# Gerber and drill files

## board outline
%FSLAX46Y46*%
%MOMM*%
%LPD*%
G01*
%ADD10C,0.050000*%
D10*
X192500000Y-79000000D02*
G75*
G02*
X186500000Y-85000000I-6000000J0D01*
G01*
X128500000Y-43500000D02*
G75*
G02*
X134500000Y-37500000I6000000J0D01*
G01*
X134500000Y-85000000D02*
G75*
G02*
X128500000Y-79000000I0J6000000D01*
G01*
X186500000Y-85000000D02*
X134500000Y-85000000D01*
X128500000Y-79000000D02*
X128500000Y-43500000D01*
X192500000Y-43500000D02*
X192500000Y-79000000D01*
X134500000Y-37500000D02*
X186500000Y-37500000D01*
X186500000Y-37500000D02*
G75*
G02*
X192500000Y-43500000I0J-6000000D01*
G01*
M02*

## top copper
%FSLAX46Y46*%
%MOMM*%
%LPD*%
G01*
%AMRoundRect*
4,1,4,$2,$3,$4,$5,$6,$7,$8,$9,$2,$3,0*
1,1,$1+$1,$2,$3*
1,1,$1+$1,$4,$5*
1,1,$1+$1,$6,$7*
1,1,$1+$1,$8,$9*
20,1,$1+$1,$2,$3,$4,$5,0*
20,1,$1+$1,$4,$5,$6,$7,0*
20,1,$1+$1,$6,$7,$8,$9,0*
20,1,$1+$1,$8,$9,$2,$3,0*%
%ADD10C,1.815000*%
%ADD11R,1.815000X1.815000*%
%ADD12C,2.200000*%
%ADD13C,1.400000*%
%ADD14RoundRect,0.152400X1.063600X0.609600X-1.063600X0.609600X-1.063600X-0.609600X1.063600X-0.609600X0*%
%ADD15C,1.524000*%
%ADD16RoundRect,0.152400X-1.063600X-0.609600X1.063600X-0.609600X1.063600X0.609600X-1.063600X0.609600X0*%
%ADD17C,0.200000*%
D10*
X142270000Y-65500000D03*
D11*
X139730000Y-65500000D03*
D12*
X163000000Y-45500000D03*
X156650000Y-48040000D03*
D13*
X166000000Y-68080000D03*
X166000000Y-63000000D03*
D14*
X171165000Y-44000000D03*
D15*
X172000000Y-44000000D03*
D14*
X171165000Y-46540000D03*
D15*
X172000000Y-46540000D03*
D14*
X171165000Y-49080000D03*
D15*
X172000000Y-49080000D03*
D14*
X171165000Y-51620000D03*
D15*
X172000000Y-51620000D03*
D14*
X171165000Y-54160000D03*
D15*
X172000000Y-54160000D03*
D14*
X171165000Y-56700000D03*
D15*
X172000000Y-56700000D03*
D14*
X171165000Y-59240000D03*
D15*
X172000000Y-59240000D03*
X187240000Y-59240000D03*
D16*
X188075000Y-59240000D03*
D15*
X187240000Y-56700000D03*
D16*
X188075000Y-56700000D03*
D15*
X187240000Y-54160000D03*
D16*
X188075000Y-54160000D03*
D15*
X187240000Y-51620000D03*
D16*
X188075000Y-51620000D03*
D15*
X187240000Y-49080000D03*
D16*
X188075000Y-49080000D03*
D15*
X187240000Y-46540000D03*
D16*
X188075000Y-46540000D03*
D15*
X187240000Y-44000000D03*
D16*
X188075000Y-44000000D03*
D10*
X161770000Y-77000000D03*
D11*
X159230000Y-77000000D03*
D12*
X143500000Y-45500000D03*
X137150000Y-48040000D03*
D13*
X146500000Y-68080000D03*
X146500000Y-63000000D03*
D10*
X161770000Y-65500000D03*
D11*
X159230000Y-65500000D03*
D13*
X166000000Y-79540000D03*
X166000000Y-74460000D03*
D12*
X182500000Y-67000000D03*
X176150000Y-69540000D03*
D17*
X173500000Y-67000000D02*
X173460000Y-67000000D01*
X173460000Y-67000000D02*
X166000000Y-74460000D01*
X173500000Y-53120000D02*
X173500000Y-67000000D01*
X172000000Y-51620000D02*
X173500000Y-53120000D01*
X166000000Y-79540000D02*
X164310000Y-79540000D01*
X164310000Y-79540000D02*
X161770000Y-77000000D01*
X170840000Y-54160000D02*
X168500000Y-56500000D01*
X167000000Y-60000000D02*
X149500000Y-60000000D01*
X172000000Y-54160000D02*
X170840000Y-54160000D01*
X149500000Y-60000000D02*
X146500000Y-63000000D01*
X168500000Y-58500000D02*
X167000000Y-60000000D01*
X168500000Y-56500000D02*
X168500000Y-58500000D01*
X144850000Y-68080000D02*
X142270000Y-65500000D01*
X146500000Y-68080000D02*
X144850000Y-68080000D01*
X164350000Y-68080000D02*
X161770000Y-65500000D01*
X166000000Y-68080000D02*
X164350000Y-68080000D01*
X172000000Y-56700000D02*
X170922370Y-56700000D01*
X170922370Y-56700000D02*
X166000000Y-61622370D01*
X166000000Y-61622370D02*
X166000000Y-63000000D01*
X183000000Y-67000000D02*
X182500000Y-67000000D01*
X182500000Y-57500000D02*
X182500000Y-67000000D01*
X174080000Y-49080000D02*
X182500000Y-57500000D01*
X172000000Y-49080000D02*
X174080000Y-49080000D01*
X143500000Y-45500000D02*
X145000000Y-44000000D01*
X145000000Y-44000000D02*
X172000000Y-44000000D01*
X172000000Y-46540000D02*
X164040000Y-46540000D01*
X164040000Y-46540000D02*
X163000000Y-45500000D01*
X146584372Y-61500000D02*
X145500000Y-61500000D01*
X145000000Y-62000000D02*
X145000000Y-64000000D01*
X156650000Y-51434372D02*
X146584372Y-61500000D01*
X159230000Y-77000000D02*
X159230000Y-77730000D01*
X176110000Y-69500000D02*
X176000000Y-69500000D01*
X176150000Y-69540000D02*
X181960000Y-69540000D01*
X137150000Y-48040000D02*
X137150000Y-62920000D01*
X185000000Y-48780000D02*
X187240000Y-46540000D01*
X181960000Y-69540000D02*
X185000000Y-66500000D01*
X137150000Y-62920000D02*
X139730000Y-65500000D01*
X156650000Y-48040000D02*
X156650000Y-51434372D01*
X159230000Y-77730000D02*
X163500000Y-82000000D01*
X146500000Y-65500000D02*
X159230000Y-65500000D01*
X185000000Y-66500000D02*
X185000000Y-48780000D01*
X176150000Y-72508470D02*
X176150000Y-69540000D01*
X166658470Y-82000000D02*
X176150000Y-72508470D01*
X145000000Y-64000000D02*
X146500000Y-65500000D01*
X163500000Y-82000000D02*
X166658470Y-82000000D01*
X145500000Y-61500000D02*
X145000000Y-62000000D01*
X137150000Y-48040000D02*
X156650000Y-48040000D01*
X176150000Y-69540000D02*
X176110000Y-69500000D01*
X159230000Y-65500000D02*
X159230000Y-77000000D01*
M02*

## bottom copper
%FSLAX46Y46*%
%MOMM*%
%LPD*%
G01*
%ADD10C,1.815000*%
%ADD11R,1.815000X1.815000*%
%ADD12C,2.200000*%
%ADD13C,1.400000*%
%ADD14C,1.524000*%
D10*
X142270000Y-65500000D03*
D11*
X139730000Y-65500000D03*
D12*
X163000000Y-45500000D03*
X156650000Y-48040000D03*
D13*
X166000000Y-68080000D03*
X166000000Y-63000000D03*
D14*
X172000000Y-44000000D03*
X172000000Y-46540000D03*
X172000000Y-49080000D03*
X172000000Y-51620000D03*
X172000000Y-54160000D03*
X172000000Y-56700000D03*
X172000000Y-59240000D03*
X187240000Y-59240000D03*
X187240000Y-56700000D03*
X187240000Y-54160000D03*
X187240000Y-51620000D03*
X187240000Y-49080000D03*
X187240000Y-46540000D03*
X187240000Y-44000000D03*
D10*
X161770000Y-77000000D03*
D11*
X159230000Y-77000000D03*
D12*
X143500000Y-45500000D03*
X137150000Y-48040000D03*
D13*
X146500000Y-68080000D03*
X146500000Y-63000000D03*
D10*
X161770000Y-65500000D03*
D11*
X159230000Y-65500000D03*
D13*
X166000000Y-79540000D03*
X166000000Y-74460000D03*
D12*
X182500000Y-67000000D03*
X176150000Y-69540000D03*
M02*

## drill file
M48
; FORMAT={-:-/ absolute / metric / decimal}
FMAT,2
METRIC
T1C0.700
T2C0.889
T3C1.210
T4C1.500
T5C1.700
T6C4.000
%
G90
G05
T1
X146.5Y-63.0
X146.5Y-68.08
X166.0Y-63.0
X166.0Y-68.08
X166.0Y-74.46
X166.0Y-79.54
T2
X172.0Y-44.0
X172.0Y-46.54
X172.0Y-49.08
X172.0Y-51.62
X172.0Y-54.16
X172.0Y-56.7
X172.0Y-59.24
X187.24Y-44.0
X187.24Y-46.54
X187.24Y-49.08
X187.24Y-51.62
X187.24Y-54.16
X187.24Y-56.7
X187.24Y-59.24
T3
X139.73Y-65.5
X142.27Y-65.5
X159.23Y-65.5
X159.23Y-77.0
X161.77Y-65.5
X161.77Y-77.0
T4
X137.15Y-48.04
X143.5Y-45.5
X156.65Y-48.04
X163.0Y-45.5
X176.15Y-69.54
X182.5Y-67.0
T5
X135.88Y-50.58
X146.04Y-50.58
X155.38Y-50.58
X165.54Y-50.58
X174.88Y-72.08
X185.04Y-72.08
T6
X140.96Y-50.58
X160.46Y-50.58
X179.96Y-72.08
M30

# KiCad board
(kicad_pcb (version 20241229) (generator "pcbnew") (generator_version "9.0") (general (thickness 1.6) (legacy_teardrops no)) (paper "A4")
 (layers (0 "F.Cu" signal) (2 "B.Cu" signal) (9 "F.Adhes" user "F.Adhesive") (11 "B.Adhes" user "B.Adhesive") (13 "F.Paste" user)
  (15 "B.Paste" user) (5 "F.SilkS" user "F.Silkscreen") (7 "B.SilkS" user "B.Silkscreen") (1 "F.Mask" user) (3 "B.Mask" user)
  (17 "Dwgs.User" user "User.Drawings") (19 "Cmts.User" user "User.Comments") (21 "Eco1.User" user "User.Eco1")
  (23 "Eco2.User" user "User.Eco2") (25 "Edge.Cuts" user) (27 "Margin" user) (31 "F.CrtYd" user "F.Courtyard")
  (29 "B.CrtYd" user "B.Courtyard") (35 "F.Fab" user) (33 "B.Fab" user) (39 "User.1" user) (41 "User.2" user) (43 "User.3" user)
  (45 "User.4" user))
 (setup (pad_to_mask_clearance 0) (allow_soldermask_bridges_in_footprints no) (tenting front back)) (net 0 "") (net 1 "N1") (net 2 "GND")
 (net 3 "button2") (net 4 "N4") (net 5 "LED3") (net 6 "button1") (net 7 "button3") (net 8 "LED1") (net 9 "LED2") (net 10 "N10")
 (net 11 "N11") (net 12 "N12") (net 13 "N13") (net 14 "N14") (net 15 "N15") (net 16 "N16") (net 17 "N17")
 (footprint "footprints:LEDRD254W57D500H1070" (layer "F.Cu") (at 141 65.5)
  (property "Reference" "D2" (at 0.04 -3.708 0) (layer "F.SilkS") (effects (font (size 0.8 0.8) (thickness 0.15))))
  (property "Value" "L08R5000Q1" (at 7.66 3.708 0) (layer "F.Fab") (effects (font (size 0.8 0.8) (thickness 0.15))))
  (pad "A" thru_hole circle (at 1.27 0) (size 1.815 1.815) (drill 1.21) (layers "*.Cu" "*.Mask") (remove_unused_layers no) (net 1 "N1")
   (solder_mask_margin 0.102))
  (pad "C" thru_hole rect (at -1.27 0) (size 1.815 1.815) (drill 1.21) (layers "*.Cu" "*.Mask") (remove_unused_layers no) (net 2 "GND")
   (solder_mask_margin 0.102)))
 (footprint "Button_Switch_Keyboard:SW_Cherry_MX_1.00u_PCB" (layer "F.Cu") (at 163 45.5)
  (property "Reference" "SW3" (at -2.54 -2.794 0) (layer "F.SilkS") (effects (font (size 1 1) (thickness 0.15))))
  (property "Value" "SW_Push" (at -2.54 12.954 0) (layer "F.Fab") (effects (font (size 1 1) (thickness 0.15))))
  (pad "" np_thru_hole circle (at -7.62 5.08) (size 1.7 1.7) (drill 1.7) (layers "*.Cu" "*.Mask"))
  (pad "" np_thru_hole circle (at -2.54 5.08) (size 4 4) (drill 4) (layers "*.Cu" "*.Mask"))
  (pad "" np_thru_hole circle (at 2.54 5.08) (size 1.7 1.7) (drill 1.7) (layers "*.Cu" "*.Mask"))
  (pad "1" thru_hole circle (at 0 0) (size 2.2 2.2) (drill 1.5) (layers "*.Cu" "*.Mask") (remove_unused_layers no) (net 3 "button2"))
  (pad "2" thru_hole circle (at -6.35 2.54) (size 2.2 2.2) (drill 1.5) (layers "*.Cu" "*.Mask") (remove_unused_layers no) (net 2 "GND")))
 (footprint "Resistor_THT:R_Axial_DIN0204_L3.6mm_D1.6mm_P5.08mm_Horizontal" (layer "F.Cu") (at 166 68.08 90)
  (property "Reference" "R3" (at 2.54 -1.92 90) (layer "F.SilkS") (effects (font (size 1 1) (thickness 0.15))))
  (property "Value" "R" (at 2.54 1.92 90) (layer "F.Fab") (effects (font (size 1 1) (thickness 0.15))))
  (pad "1" thru_hole circle (at 0 0 90) (size 1.4 1.4) (drill 0.7) (layers "*.Cu" "*.Mask") (remove_unused_layers no) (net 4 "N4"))
  (pad "2" thru_hole circle (at 5.08 0 90) (size 1.4 1.4) (drill 0.7) (layers "*.Cu" "*.Mask") (remove_unused_layers no) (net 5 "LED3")))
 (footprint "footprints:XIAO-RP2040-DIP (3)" (layer "F.Cu") (at 179.62 51.62)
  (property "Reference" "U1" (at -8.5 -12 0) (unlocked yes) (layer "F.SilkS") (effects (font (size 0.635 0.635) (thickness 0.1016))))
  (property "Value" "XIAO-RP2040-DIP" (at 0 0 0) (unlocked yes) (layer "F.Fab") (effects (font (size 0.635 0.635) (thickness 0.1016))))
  (pad "1" smd roundrect (at -8.455 -7.62 180) (size 2.432 1.524) (layers "F.Cu" "F.Mask") (roundrect_rratio 0.1) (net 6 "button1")
   (thermal_bridge_angle 45))
  (pad "1" thru_hole circle (at -7.62 -7.62 180) (size 1.524 1.524) (drill 0.889) (layers "*.Cu" "*.Mask") (remove_unused_layers no)
   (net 6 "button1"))
  (pad "2" smd roundrect (at -8.455 -5.08 180) (size 2.432 1.524) (layers "F.Cu" "F.Mask") (roundrect_rratio 0.1) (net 3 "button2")
   (thermal_bridge_angle 45))
  (pad "2" thru_hole circle (at -7.62 -5.08 180) (size 1.524 1.524) (drill 0.889) (layers "*.Cu" "*.Mask") (remove_unused_layers no)
   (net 3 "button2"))
  (pad "3" smd roundrect (at -8.455 -2.54 180) (size 2.432 1.524) (layers "F.Cu" "F.Mask") (roundrect_rratio 0.1) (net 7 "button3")
   (thermal_bridge_angle 45))
  (pad "3" thru_hole circle (at -7.62 -2.54 180) (size 1.524 1.524) (drill 0.889) (layers "*.Cu" "*.Mask") (remove_unused_layers no)
   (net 7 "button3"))
  (pad "4" smd roundrect (at -8.455 0 180) (size 2.432 1.524) (layers "F.Cu" "F.Mask") (roundrect_rratio 0.1) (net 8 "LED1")
   (thermal_bridge_angle 45))
  (pad "4" thru_hole circle (at -7.62 0 180) (size 1.524 1.524) (drill 0.889) (layers "*.Cu" "*.Mask") (remove_unused_layers no)
   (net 8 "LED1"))
  (pad "5" smd roundrect (at -8.455 2.54 180) (size 2.432 1.524) (layers "F.Cu" "F.Mask") (roundrect_rratio 0.1) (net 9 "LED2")
   (thermal_bridge_angle 45))
  (pad "5" thru_hole circle (at -7.62 2.54 180) (size 1.524 1.524) (drill 0.889) (layers "*.Cu" "*.Mask") (remove_unused_layers no)
   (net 9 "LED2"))
  (pad "6" smd roundrect (at -8.455 5.08 180) (size 2.432 1.524) (layers "F.Cu" "F.Mask") (roundrect_rratio 0.1) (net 5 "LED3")
   (thermal_bridge_angle 45))
  (pad "6" thru_hole circle (at -7.62 5.08 180) (size 1.524 1.524) (drill 0.889) (layers "*.Cu" "*.Mask") (remove_unused_layers no)
   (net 5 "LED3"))
  (pad "7" smd roundrect (at -8.455 7.62 180) (size 2.432 1.524) (layers "F.Cu" "F.Mask") (roundrect_rratio 0.1) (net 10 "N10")
   (thermal_bridge_angle 45))
  (pad "7" thru_hole circle (at -7.62 7.62 180) (size 1.524 1.524) (drill 0.889) (layers "*.Cu" "*.Mask") (remove_unused_layers no)
   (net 10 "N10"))
  (pad "8" thru_hole circle (at 7.62 7.62) (size 1.524 1.524) (drill 0.889) (layers "*.Cu" "*.Mask") (remove_unused_layers no)
   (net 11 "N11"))
  (pad "8" smd roundrect (at 8.455 7.62) (size 2.432 1.524) (layers "F.Cu" "F.Mask") (roundrect_rratio 0.1) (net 11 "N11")
   (thermal_bridge_angle 45))
  (pad "9" thru_hole circle (at 7.62 5.08) (size 1.524 1.524) (drill 0.889) (layers "*.Cu" "*.Mask") (remove_unused_layers no)
   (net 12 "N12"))
  (pad "9" smd roundrect (at 8.455 5.08) (size 2.432 1.524) (layers "F.Cu" "F.Mask") (roundrect_rratio 0.1) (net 12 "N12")
   (thermal_bridge_angle 45))
  (pad "10" thru_hole circle (at 7.62 2.54) (size 1.524 1.524) (drill 0.889) (layers "*.Cu" "*.Mask") (remove_unused_layers no)
   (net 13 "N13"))
  (pad "10" smd roundrect (at 8.455 2.54) (size 2.432 1.524) (layers "F.Cu" "F.Mask") (roundrect_rratio 0.1) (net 13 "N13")
   (thermal_bridge_angle 45))
  (pad "11" thru_hole circle (at 7.62 0) (size 1.524 1.524) (drill 0.889) (layers "*.Cu" "*.Mask") (remove_unused_layers no) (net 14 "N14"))
  (pad "11" smd roundrect (at 8.455 0) (size 2.432 1.524) (layers "F.Cu" "F.Mask") (roundrect_rratio 0.1) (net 14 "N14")
   (thermal_bridge_angle 45))
  (pad "12" thru_hole circle (at 7.62 -2.54) (size 1.524 1.524) (drill 0.889) (layers "*.Cu" "*.Mask") (remove_unused_layers no)
   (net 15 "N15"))
  (pad "12" smd roundrect (at 8.455 -2.54) (size 2.432 1.524) (layers "F.Cu" "F.Mask") (roundrect_rratio 0.1) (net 15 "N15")
   (thermal_bridge_angle 45))
  (pad "13" thru_hole circle (at 7.62 -5.08) (size 1.524 1.524) (drill 0.889) (layers "*.Cu" "*.Mask") (remove_unused_layers no)
   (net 2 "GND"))
  (pad "13" smd roundrect (at 8.455 -5.08) (size 2.432 1.524) (layers "F.Cu" "F.Mask") (roundrect_rratio 0.1) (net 2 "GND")
   (thermal_bridge_angle 45))
  (pad "14" thru_hole circle (at 7.62 -7.62) (size 1.524 1.524) (drill 0.889) (layers "*.Cu" "*.Mask") (remove_unused_layers no)
   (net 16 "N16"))
  (pad "14" smd roundrect (at 8.455 -7.62) (size 2.432 1.524) (layers "F.Cu" "F.Mask") (roundrect_rratio 0.1) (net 16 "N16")
   (thermal_bridge_angle 45)))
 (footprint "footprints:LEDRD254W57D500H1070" (layer "F.Cu") (at 160.5 77)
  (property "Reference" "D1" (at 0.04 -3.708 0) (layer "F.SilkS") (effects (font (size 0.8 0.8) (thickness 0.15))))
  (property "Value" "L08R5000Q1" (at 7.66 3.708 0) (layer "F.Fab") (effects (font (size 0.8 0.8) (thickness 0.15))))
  (pad "A" thru_hole circle (at 1.27 0) (size 1.815 1.815) (drill 1.21) (layers "*.Cu" "*.Mask") (remove_unused_layers no) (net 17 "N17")
   (solder_mask_margin 0.102))
  (pad "C" thru_hole rect (at -1.27 0) (size 1.815 1.815) (drill 1.21) (layers "*.Cu" "*.Mask") (remove_unused_layers no) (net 2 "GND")
   (solder_mask_margin 0.102)))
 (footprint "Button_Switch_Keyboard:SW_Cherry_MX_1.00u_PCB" (layer "F.Cu") (at 143.5 45.5)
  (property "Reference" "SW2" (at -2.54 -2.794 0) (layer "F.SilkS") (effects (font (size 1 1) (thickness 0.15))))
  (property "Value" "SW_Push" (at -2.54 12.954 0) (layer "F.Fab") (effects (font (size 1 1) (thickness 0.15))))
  (pad "" np_thru_hole circle (at -7.62 5.08) (size 1.7 1.7) (drill 1.7) (layers "*.Cu" "*.Mask"))
  (pad "" np_thru_hole circle (at -2.54 5.08) (size 4 4) (drill 4) (layers "*.Cu" "*.Mask"))
  (pad "" np_thru_hole circle (at 2.54 5.08) (size 1.7 1.7) (drill 1.7) (layers "*.Cu" "*.Mask"))
  (pad "1" thru_hole circle (at 0 0) (size 2.2 2.2) (drill 1.5) (layers "*.Cu" "*.Mask") (remove_unused_layers no) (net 6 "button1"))
  (pad "2" thru_hole circle (at -6.35 2.54) (size 2.2 2.2) (drill 1.5) (layers "*.Cu" "*.Mask") (remove_unused_layers no) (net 2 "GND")))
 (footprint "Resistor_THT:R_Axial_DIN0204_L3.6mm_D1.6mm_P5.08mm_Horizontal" (layer "F.Cu") (at 146.5 68.08 90)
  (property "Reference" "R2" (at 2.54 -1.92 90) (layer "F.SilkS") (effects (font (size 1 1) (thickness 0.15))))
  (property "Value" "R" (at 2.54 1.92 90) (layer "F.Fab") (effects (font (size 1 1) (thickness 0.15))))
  (pad "1" thru_hole circle (at 0 0 90) (size 1.4 1.4) (drill 0.7) (layers "*.Cu" "*.Mask") (remove_unused_layers no) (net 1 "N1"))
  (pad "2" thru_hole circle (at 5.08 0 90) (size 1.4 1.4) (drill 0.7) (layers "*.Cu" "*.Mask") (remove_unused_layers no) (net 9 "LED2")))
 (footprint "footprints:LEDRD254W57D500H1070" (layer "F.Cu") (at 160.5 65.5)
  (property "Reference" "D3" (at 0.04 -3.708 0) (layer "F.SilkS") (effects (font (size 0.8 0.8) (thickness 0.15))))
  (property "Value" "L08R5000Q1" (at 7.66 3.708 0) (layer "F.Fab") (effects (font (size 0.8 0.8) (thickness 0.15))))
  (pad "A" thru_hole circle (at 1.27 0) (size 1.815 1.815) (drill 1.21) (layers "*.Cu" "*.Mask") (remove_unused_layers no) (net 4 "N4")
   (solder_mask_margin 0.102))
  (pad "C" thru_hole rect (at -1.27 0) (size 1.815 1.815) (drill 1.21) (layers "*.Cu" "*.Mask") (remove_unused_layers no) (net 2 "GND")
   (solder_mask_margin 0.102)))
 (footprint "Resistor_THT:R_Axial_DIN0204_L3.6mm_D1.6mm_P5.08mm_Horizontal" (layer "F.Cu") (at 166 79.54 90)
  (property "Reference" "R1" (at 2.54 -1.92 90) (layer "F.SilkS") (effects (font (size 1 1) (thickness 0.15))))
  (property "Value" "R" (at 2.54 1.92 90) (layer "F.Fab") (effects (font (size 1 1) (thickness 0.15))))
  (pad "1" thru_hole circle (at 0 0 90) (size 1.4 1.4) (drill 0.7) (layers "*.Cu" "*.Mask") (remove_unused_layers no) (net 17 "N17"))
  (pad "2" thru_hole circle (at 5.08 0 90) (size 1.4 1.4) (drill 0.7) (layers "*.Cu" "*.Mask") (remove_unused_layers no) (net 8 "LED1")))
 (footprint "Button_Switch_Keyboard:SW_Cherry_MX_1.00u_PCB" (layer "F.Cu") (at 182.5 67)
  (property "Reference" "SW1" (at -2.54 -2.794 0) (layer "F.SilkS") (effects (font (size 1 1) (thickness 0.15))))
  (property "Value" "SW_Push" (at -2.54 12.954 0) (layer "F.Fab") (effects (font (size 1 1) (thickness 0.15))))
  (pad "" np_thru_hole circle (at -7.62 5.08) (size 1.7 1.7) (drill 1.7) (layers "*.Cu" "*.Mask"))
  (pad "" np_thru_hole circle (at -2.54 5.08) (size 4 4) (drill 4) (layers "*.Cu" "*.Mask"))
  (pad "" np_thru_hole circle (at 2.54 5.08) (size 1.7 1.7) (drill 1.7) (layers "*.Cu" "*.Mask"))
  (pad "1" thru_hole circle (at 0 0) (size 2.2 2.2) (drill 1.5) (layers "*.Cu" "*.Mask") (remove_unused_layers no) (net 7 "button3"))
  (pad "2" thru_hole circle (at -6.35 2.54) (size 2.2 2.2) (drill 1.5) (layers "*.Cu" "*.Mask") (remove_unused_layers no) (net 2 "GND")))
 (gr_arc (start 192.5 79) (mid 190.742641 83.242641) (end 186.5 85) (stroke (width 0.05) (type default)) (layer "Edge.Cuts"))
 (gr_arc (start 128.5 43.5) (mid 130.257359 39.257359) (end 134.5 37.5) (stroke (width 0.05) (type default)) (layer "Edge.Cuts"))
 (gr_arc (start 134.5 85) (mid 130.257359 83.242641) (end 128.5 79) (stroke (width 0.05) (type default)) (layer "Edge.Cuts"))
 (gr_line (start 186.5 85) (end 134.5 85) (stroke (width 0.05) (type default)) (layer "Edge.Cuts"))
 (gr_line (start 128.5 79) (end 128.5 43.5) (stroke (width 0.05) (type default)) (layer "Edge.Cuts"))
 (gr_line (start 192.5 43.5) (end 192.5 79) (stroke (width 0.05) (type default)) (layer "Edge.Cuts"))
 (gr_line (start 134.5 37.5) (end 186.5 37.5) (stroke (width 0.05) (type default)) (layer "Edge.Cuts"))
 (gr_arc (start 186.5 37.5) (mid 190.742641 39.257359) (end 192.5 43.5) (stroke (width 0.05) (type default)) (layer "Edge.Cuts"))
 (segment (start 173.5 67) (end 173.46 67) (width 0.2) (layer "F.Cu") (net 8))
 (segment (start 173.46 67) (end 166 74.46) (width 0.2) (layer "F.Cu") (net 8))
 (segment (start 173.5 53.12) (end 173.5 67) (width 0.2) (layer "F.Cu") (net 8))
 (segment (start 172 51.62) (end 173.5 53.12) (width 0.2) (layer "F.Cu") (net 8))
 (segment (start 166 79.54) (end 164.31 79.54) (width 0.2) (layer "F.Cu") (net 17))
 (segment (start 164.31 79.54) (end 161.77 77) (width 0.2) (layer "F.Cu") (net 17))
 (segment (start 170.84 54.16) (end 168.5 56.5) (width 0.2) (layer "F.Cu") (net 9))
 (segment (start 167 60) (end 149.5 60) (width 0.2) (layer "F.Cu") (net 9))
 (segment (start 172 54.16) (end 170.84 54.16) (width 0.2) (layer "F.Cu") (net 9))
 (segment (start 149.5 60) (end 146.5 63) (width 0.2) (layer "F.Cu") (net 9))
 (segment (start 168.5 58.5) (end 167 60) (width 0.2) (layer "F.Cu") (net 9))
 (segment (start 168.5 56.5) (end 168.5 58.5) (width 0.2) (layer "F.Cu") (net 9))
 (segment (start 144.85 68.08) (end 142.27 65.5) (width 0.2) (layer "F.Cu") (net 1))
 (segment (start 146.5 68.08) (end 144.85 68.08) (width 0.2) (layer "F.Cu") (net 1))
 (segment (start 164.35 68.08) (end 161.77 65.5) (width 0.2) (layer "F.Cu") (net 4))
 (segment (start 166 68.08) (end 164.35 68.08) (width 0.2) (layer "F.Cu") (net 4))
 (segment (start 172 56.7) (end 170.92237 56.7) (width 0.2) (layer "F.Cu") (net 5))
 (segment (start 170.92237 56.7) (end 166 61.62237) (width 0.2) (layer "F.Cu") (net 5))
 (segment (start 166 61.62237) (end 166 63) (width 0.2) (layer "F.Cu") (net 5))
 (segment (start 183 67) (end 182.5 67) (width 0.2) (layer "F.Cu") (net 7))
 (segment (start 182.5 57.5) (end 182.5 67) (width 0.2) (layer "F.Cu") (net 7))
 (segment (start 174.08 49.08) (end 182.5 57.5) (width 0.2) (layer "F.Cu") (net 7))
 (segment (start 172 49.08) (end 174.08 49.08) (width 0.2) (layer "F.Cu") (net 7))
 (segment (start 143.5 45.5) (end 145 44) (width 0.2) (layer "F.Cu") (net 6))
 (segment (start 145 44) (end 172 44) (width 0.2) (layer "F.Cu") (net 6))
 (segment (start 172 46.54) (end 164.04 46.54) (width 0.2) (layer "F.Cu") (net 3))
 (segment (start 164.04 46.54) (end 163 45.5) (width 0.2) (layer "F.Cu") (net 3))
 (segment (start 146.584372 61.5) (end 145.5 61.5) (width 0.2) (layer "F.Cu") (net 2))
 (segment (start 145 62) (end 145 64) (width 0.2) (layer "F.Cu") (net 2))
 (segment (start 156.65 51.434372) (end 146.584372 61.5) (width 0.2) (layer "F.Cu") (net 2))
 (segment (start 159.23 77) (end 159.23 77.73) (width 0.2) (layer "F.Cu") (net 2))
 (segment (start 176.11 69.5) (end 176 69.5) (width 0.2) (layer "F.Cu") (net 2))
 (segment (start 176.15 69.54) (end 181.96 69.54) (width 0.2) (layer "F.Cu") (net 2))
 (segment (start 137.15 48.04) (end 137.15 62.92) (width 0.2) (layer "F.Cu") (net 2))
 (segment (start 185 48.78) (end 187.24 46.54) (width 0.2) (layer "F.Cu") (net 2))
 (segment (start 181.96 69.54) (end 185 66.5) (width 0.2) (layer "F.Cu") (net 2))
 (segment (start 137.15 62.92) (end 139.73 65.5) (width 0.2) (layer "F.Cu") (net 2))
 (segment (start 156.65 48.04) (end 156.65 51.434372) (width 0.2) (layer "F.Cu") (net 2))
 (segment (start 159.23 77.73) (end 163.5 82) (width 0.2) (layer "F.Cu") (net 2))
 (segment (start 146.5 65.5) (end 159.23 65.5) (width 0.2) (layer "F.Cu") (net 2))
 (segment (start 185 66.5) (end 185 48.78) (width 0.2) (layer "F.Cu") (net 2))
 (segment (start 176.15 72.50847) (end 176.15 69.54) (width 0.2) (layer "F.Cu") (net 2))
 (segment (start 166.65847 82) (end 176.15 72.50847) (width 0.2) (layer "F.Cu") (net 2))
 (segment (start 145 64) (end 146.5 65.5) (width 0.2) (layer "F.Cu") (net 2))
 (segment (start 163.5 82) (end 166.65847 82) (width 0.2) (layer "F.Cu") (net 2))
 (segment (start 145.5 61.5) (end 145 62) (width 0.2) (layer "F.Cu") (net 2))
 (segment (start 137.15 48.04) (end 156.65 48.04) (width 0.2) (layer "F.Cu") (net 2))
 (segment (start 176.15 69.54) (end 176.11 69.5) (width 0.2) (layer "F.Cu") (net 2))
 (segment (start 159.23 65.5) (end 159.23 77) (width 0.2) (layer "F.Cu") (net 2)))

